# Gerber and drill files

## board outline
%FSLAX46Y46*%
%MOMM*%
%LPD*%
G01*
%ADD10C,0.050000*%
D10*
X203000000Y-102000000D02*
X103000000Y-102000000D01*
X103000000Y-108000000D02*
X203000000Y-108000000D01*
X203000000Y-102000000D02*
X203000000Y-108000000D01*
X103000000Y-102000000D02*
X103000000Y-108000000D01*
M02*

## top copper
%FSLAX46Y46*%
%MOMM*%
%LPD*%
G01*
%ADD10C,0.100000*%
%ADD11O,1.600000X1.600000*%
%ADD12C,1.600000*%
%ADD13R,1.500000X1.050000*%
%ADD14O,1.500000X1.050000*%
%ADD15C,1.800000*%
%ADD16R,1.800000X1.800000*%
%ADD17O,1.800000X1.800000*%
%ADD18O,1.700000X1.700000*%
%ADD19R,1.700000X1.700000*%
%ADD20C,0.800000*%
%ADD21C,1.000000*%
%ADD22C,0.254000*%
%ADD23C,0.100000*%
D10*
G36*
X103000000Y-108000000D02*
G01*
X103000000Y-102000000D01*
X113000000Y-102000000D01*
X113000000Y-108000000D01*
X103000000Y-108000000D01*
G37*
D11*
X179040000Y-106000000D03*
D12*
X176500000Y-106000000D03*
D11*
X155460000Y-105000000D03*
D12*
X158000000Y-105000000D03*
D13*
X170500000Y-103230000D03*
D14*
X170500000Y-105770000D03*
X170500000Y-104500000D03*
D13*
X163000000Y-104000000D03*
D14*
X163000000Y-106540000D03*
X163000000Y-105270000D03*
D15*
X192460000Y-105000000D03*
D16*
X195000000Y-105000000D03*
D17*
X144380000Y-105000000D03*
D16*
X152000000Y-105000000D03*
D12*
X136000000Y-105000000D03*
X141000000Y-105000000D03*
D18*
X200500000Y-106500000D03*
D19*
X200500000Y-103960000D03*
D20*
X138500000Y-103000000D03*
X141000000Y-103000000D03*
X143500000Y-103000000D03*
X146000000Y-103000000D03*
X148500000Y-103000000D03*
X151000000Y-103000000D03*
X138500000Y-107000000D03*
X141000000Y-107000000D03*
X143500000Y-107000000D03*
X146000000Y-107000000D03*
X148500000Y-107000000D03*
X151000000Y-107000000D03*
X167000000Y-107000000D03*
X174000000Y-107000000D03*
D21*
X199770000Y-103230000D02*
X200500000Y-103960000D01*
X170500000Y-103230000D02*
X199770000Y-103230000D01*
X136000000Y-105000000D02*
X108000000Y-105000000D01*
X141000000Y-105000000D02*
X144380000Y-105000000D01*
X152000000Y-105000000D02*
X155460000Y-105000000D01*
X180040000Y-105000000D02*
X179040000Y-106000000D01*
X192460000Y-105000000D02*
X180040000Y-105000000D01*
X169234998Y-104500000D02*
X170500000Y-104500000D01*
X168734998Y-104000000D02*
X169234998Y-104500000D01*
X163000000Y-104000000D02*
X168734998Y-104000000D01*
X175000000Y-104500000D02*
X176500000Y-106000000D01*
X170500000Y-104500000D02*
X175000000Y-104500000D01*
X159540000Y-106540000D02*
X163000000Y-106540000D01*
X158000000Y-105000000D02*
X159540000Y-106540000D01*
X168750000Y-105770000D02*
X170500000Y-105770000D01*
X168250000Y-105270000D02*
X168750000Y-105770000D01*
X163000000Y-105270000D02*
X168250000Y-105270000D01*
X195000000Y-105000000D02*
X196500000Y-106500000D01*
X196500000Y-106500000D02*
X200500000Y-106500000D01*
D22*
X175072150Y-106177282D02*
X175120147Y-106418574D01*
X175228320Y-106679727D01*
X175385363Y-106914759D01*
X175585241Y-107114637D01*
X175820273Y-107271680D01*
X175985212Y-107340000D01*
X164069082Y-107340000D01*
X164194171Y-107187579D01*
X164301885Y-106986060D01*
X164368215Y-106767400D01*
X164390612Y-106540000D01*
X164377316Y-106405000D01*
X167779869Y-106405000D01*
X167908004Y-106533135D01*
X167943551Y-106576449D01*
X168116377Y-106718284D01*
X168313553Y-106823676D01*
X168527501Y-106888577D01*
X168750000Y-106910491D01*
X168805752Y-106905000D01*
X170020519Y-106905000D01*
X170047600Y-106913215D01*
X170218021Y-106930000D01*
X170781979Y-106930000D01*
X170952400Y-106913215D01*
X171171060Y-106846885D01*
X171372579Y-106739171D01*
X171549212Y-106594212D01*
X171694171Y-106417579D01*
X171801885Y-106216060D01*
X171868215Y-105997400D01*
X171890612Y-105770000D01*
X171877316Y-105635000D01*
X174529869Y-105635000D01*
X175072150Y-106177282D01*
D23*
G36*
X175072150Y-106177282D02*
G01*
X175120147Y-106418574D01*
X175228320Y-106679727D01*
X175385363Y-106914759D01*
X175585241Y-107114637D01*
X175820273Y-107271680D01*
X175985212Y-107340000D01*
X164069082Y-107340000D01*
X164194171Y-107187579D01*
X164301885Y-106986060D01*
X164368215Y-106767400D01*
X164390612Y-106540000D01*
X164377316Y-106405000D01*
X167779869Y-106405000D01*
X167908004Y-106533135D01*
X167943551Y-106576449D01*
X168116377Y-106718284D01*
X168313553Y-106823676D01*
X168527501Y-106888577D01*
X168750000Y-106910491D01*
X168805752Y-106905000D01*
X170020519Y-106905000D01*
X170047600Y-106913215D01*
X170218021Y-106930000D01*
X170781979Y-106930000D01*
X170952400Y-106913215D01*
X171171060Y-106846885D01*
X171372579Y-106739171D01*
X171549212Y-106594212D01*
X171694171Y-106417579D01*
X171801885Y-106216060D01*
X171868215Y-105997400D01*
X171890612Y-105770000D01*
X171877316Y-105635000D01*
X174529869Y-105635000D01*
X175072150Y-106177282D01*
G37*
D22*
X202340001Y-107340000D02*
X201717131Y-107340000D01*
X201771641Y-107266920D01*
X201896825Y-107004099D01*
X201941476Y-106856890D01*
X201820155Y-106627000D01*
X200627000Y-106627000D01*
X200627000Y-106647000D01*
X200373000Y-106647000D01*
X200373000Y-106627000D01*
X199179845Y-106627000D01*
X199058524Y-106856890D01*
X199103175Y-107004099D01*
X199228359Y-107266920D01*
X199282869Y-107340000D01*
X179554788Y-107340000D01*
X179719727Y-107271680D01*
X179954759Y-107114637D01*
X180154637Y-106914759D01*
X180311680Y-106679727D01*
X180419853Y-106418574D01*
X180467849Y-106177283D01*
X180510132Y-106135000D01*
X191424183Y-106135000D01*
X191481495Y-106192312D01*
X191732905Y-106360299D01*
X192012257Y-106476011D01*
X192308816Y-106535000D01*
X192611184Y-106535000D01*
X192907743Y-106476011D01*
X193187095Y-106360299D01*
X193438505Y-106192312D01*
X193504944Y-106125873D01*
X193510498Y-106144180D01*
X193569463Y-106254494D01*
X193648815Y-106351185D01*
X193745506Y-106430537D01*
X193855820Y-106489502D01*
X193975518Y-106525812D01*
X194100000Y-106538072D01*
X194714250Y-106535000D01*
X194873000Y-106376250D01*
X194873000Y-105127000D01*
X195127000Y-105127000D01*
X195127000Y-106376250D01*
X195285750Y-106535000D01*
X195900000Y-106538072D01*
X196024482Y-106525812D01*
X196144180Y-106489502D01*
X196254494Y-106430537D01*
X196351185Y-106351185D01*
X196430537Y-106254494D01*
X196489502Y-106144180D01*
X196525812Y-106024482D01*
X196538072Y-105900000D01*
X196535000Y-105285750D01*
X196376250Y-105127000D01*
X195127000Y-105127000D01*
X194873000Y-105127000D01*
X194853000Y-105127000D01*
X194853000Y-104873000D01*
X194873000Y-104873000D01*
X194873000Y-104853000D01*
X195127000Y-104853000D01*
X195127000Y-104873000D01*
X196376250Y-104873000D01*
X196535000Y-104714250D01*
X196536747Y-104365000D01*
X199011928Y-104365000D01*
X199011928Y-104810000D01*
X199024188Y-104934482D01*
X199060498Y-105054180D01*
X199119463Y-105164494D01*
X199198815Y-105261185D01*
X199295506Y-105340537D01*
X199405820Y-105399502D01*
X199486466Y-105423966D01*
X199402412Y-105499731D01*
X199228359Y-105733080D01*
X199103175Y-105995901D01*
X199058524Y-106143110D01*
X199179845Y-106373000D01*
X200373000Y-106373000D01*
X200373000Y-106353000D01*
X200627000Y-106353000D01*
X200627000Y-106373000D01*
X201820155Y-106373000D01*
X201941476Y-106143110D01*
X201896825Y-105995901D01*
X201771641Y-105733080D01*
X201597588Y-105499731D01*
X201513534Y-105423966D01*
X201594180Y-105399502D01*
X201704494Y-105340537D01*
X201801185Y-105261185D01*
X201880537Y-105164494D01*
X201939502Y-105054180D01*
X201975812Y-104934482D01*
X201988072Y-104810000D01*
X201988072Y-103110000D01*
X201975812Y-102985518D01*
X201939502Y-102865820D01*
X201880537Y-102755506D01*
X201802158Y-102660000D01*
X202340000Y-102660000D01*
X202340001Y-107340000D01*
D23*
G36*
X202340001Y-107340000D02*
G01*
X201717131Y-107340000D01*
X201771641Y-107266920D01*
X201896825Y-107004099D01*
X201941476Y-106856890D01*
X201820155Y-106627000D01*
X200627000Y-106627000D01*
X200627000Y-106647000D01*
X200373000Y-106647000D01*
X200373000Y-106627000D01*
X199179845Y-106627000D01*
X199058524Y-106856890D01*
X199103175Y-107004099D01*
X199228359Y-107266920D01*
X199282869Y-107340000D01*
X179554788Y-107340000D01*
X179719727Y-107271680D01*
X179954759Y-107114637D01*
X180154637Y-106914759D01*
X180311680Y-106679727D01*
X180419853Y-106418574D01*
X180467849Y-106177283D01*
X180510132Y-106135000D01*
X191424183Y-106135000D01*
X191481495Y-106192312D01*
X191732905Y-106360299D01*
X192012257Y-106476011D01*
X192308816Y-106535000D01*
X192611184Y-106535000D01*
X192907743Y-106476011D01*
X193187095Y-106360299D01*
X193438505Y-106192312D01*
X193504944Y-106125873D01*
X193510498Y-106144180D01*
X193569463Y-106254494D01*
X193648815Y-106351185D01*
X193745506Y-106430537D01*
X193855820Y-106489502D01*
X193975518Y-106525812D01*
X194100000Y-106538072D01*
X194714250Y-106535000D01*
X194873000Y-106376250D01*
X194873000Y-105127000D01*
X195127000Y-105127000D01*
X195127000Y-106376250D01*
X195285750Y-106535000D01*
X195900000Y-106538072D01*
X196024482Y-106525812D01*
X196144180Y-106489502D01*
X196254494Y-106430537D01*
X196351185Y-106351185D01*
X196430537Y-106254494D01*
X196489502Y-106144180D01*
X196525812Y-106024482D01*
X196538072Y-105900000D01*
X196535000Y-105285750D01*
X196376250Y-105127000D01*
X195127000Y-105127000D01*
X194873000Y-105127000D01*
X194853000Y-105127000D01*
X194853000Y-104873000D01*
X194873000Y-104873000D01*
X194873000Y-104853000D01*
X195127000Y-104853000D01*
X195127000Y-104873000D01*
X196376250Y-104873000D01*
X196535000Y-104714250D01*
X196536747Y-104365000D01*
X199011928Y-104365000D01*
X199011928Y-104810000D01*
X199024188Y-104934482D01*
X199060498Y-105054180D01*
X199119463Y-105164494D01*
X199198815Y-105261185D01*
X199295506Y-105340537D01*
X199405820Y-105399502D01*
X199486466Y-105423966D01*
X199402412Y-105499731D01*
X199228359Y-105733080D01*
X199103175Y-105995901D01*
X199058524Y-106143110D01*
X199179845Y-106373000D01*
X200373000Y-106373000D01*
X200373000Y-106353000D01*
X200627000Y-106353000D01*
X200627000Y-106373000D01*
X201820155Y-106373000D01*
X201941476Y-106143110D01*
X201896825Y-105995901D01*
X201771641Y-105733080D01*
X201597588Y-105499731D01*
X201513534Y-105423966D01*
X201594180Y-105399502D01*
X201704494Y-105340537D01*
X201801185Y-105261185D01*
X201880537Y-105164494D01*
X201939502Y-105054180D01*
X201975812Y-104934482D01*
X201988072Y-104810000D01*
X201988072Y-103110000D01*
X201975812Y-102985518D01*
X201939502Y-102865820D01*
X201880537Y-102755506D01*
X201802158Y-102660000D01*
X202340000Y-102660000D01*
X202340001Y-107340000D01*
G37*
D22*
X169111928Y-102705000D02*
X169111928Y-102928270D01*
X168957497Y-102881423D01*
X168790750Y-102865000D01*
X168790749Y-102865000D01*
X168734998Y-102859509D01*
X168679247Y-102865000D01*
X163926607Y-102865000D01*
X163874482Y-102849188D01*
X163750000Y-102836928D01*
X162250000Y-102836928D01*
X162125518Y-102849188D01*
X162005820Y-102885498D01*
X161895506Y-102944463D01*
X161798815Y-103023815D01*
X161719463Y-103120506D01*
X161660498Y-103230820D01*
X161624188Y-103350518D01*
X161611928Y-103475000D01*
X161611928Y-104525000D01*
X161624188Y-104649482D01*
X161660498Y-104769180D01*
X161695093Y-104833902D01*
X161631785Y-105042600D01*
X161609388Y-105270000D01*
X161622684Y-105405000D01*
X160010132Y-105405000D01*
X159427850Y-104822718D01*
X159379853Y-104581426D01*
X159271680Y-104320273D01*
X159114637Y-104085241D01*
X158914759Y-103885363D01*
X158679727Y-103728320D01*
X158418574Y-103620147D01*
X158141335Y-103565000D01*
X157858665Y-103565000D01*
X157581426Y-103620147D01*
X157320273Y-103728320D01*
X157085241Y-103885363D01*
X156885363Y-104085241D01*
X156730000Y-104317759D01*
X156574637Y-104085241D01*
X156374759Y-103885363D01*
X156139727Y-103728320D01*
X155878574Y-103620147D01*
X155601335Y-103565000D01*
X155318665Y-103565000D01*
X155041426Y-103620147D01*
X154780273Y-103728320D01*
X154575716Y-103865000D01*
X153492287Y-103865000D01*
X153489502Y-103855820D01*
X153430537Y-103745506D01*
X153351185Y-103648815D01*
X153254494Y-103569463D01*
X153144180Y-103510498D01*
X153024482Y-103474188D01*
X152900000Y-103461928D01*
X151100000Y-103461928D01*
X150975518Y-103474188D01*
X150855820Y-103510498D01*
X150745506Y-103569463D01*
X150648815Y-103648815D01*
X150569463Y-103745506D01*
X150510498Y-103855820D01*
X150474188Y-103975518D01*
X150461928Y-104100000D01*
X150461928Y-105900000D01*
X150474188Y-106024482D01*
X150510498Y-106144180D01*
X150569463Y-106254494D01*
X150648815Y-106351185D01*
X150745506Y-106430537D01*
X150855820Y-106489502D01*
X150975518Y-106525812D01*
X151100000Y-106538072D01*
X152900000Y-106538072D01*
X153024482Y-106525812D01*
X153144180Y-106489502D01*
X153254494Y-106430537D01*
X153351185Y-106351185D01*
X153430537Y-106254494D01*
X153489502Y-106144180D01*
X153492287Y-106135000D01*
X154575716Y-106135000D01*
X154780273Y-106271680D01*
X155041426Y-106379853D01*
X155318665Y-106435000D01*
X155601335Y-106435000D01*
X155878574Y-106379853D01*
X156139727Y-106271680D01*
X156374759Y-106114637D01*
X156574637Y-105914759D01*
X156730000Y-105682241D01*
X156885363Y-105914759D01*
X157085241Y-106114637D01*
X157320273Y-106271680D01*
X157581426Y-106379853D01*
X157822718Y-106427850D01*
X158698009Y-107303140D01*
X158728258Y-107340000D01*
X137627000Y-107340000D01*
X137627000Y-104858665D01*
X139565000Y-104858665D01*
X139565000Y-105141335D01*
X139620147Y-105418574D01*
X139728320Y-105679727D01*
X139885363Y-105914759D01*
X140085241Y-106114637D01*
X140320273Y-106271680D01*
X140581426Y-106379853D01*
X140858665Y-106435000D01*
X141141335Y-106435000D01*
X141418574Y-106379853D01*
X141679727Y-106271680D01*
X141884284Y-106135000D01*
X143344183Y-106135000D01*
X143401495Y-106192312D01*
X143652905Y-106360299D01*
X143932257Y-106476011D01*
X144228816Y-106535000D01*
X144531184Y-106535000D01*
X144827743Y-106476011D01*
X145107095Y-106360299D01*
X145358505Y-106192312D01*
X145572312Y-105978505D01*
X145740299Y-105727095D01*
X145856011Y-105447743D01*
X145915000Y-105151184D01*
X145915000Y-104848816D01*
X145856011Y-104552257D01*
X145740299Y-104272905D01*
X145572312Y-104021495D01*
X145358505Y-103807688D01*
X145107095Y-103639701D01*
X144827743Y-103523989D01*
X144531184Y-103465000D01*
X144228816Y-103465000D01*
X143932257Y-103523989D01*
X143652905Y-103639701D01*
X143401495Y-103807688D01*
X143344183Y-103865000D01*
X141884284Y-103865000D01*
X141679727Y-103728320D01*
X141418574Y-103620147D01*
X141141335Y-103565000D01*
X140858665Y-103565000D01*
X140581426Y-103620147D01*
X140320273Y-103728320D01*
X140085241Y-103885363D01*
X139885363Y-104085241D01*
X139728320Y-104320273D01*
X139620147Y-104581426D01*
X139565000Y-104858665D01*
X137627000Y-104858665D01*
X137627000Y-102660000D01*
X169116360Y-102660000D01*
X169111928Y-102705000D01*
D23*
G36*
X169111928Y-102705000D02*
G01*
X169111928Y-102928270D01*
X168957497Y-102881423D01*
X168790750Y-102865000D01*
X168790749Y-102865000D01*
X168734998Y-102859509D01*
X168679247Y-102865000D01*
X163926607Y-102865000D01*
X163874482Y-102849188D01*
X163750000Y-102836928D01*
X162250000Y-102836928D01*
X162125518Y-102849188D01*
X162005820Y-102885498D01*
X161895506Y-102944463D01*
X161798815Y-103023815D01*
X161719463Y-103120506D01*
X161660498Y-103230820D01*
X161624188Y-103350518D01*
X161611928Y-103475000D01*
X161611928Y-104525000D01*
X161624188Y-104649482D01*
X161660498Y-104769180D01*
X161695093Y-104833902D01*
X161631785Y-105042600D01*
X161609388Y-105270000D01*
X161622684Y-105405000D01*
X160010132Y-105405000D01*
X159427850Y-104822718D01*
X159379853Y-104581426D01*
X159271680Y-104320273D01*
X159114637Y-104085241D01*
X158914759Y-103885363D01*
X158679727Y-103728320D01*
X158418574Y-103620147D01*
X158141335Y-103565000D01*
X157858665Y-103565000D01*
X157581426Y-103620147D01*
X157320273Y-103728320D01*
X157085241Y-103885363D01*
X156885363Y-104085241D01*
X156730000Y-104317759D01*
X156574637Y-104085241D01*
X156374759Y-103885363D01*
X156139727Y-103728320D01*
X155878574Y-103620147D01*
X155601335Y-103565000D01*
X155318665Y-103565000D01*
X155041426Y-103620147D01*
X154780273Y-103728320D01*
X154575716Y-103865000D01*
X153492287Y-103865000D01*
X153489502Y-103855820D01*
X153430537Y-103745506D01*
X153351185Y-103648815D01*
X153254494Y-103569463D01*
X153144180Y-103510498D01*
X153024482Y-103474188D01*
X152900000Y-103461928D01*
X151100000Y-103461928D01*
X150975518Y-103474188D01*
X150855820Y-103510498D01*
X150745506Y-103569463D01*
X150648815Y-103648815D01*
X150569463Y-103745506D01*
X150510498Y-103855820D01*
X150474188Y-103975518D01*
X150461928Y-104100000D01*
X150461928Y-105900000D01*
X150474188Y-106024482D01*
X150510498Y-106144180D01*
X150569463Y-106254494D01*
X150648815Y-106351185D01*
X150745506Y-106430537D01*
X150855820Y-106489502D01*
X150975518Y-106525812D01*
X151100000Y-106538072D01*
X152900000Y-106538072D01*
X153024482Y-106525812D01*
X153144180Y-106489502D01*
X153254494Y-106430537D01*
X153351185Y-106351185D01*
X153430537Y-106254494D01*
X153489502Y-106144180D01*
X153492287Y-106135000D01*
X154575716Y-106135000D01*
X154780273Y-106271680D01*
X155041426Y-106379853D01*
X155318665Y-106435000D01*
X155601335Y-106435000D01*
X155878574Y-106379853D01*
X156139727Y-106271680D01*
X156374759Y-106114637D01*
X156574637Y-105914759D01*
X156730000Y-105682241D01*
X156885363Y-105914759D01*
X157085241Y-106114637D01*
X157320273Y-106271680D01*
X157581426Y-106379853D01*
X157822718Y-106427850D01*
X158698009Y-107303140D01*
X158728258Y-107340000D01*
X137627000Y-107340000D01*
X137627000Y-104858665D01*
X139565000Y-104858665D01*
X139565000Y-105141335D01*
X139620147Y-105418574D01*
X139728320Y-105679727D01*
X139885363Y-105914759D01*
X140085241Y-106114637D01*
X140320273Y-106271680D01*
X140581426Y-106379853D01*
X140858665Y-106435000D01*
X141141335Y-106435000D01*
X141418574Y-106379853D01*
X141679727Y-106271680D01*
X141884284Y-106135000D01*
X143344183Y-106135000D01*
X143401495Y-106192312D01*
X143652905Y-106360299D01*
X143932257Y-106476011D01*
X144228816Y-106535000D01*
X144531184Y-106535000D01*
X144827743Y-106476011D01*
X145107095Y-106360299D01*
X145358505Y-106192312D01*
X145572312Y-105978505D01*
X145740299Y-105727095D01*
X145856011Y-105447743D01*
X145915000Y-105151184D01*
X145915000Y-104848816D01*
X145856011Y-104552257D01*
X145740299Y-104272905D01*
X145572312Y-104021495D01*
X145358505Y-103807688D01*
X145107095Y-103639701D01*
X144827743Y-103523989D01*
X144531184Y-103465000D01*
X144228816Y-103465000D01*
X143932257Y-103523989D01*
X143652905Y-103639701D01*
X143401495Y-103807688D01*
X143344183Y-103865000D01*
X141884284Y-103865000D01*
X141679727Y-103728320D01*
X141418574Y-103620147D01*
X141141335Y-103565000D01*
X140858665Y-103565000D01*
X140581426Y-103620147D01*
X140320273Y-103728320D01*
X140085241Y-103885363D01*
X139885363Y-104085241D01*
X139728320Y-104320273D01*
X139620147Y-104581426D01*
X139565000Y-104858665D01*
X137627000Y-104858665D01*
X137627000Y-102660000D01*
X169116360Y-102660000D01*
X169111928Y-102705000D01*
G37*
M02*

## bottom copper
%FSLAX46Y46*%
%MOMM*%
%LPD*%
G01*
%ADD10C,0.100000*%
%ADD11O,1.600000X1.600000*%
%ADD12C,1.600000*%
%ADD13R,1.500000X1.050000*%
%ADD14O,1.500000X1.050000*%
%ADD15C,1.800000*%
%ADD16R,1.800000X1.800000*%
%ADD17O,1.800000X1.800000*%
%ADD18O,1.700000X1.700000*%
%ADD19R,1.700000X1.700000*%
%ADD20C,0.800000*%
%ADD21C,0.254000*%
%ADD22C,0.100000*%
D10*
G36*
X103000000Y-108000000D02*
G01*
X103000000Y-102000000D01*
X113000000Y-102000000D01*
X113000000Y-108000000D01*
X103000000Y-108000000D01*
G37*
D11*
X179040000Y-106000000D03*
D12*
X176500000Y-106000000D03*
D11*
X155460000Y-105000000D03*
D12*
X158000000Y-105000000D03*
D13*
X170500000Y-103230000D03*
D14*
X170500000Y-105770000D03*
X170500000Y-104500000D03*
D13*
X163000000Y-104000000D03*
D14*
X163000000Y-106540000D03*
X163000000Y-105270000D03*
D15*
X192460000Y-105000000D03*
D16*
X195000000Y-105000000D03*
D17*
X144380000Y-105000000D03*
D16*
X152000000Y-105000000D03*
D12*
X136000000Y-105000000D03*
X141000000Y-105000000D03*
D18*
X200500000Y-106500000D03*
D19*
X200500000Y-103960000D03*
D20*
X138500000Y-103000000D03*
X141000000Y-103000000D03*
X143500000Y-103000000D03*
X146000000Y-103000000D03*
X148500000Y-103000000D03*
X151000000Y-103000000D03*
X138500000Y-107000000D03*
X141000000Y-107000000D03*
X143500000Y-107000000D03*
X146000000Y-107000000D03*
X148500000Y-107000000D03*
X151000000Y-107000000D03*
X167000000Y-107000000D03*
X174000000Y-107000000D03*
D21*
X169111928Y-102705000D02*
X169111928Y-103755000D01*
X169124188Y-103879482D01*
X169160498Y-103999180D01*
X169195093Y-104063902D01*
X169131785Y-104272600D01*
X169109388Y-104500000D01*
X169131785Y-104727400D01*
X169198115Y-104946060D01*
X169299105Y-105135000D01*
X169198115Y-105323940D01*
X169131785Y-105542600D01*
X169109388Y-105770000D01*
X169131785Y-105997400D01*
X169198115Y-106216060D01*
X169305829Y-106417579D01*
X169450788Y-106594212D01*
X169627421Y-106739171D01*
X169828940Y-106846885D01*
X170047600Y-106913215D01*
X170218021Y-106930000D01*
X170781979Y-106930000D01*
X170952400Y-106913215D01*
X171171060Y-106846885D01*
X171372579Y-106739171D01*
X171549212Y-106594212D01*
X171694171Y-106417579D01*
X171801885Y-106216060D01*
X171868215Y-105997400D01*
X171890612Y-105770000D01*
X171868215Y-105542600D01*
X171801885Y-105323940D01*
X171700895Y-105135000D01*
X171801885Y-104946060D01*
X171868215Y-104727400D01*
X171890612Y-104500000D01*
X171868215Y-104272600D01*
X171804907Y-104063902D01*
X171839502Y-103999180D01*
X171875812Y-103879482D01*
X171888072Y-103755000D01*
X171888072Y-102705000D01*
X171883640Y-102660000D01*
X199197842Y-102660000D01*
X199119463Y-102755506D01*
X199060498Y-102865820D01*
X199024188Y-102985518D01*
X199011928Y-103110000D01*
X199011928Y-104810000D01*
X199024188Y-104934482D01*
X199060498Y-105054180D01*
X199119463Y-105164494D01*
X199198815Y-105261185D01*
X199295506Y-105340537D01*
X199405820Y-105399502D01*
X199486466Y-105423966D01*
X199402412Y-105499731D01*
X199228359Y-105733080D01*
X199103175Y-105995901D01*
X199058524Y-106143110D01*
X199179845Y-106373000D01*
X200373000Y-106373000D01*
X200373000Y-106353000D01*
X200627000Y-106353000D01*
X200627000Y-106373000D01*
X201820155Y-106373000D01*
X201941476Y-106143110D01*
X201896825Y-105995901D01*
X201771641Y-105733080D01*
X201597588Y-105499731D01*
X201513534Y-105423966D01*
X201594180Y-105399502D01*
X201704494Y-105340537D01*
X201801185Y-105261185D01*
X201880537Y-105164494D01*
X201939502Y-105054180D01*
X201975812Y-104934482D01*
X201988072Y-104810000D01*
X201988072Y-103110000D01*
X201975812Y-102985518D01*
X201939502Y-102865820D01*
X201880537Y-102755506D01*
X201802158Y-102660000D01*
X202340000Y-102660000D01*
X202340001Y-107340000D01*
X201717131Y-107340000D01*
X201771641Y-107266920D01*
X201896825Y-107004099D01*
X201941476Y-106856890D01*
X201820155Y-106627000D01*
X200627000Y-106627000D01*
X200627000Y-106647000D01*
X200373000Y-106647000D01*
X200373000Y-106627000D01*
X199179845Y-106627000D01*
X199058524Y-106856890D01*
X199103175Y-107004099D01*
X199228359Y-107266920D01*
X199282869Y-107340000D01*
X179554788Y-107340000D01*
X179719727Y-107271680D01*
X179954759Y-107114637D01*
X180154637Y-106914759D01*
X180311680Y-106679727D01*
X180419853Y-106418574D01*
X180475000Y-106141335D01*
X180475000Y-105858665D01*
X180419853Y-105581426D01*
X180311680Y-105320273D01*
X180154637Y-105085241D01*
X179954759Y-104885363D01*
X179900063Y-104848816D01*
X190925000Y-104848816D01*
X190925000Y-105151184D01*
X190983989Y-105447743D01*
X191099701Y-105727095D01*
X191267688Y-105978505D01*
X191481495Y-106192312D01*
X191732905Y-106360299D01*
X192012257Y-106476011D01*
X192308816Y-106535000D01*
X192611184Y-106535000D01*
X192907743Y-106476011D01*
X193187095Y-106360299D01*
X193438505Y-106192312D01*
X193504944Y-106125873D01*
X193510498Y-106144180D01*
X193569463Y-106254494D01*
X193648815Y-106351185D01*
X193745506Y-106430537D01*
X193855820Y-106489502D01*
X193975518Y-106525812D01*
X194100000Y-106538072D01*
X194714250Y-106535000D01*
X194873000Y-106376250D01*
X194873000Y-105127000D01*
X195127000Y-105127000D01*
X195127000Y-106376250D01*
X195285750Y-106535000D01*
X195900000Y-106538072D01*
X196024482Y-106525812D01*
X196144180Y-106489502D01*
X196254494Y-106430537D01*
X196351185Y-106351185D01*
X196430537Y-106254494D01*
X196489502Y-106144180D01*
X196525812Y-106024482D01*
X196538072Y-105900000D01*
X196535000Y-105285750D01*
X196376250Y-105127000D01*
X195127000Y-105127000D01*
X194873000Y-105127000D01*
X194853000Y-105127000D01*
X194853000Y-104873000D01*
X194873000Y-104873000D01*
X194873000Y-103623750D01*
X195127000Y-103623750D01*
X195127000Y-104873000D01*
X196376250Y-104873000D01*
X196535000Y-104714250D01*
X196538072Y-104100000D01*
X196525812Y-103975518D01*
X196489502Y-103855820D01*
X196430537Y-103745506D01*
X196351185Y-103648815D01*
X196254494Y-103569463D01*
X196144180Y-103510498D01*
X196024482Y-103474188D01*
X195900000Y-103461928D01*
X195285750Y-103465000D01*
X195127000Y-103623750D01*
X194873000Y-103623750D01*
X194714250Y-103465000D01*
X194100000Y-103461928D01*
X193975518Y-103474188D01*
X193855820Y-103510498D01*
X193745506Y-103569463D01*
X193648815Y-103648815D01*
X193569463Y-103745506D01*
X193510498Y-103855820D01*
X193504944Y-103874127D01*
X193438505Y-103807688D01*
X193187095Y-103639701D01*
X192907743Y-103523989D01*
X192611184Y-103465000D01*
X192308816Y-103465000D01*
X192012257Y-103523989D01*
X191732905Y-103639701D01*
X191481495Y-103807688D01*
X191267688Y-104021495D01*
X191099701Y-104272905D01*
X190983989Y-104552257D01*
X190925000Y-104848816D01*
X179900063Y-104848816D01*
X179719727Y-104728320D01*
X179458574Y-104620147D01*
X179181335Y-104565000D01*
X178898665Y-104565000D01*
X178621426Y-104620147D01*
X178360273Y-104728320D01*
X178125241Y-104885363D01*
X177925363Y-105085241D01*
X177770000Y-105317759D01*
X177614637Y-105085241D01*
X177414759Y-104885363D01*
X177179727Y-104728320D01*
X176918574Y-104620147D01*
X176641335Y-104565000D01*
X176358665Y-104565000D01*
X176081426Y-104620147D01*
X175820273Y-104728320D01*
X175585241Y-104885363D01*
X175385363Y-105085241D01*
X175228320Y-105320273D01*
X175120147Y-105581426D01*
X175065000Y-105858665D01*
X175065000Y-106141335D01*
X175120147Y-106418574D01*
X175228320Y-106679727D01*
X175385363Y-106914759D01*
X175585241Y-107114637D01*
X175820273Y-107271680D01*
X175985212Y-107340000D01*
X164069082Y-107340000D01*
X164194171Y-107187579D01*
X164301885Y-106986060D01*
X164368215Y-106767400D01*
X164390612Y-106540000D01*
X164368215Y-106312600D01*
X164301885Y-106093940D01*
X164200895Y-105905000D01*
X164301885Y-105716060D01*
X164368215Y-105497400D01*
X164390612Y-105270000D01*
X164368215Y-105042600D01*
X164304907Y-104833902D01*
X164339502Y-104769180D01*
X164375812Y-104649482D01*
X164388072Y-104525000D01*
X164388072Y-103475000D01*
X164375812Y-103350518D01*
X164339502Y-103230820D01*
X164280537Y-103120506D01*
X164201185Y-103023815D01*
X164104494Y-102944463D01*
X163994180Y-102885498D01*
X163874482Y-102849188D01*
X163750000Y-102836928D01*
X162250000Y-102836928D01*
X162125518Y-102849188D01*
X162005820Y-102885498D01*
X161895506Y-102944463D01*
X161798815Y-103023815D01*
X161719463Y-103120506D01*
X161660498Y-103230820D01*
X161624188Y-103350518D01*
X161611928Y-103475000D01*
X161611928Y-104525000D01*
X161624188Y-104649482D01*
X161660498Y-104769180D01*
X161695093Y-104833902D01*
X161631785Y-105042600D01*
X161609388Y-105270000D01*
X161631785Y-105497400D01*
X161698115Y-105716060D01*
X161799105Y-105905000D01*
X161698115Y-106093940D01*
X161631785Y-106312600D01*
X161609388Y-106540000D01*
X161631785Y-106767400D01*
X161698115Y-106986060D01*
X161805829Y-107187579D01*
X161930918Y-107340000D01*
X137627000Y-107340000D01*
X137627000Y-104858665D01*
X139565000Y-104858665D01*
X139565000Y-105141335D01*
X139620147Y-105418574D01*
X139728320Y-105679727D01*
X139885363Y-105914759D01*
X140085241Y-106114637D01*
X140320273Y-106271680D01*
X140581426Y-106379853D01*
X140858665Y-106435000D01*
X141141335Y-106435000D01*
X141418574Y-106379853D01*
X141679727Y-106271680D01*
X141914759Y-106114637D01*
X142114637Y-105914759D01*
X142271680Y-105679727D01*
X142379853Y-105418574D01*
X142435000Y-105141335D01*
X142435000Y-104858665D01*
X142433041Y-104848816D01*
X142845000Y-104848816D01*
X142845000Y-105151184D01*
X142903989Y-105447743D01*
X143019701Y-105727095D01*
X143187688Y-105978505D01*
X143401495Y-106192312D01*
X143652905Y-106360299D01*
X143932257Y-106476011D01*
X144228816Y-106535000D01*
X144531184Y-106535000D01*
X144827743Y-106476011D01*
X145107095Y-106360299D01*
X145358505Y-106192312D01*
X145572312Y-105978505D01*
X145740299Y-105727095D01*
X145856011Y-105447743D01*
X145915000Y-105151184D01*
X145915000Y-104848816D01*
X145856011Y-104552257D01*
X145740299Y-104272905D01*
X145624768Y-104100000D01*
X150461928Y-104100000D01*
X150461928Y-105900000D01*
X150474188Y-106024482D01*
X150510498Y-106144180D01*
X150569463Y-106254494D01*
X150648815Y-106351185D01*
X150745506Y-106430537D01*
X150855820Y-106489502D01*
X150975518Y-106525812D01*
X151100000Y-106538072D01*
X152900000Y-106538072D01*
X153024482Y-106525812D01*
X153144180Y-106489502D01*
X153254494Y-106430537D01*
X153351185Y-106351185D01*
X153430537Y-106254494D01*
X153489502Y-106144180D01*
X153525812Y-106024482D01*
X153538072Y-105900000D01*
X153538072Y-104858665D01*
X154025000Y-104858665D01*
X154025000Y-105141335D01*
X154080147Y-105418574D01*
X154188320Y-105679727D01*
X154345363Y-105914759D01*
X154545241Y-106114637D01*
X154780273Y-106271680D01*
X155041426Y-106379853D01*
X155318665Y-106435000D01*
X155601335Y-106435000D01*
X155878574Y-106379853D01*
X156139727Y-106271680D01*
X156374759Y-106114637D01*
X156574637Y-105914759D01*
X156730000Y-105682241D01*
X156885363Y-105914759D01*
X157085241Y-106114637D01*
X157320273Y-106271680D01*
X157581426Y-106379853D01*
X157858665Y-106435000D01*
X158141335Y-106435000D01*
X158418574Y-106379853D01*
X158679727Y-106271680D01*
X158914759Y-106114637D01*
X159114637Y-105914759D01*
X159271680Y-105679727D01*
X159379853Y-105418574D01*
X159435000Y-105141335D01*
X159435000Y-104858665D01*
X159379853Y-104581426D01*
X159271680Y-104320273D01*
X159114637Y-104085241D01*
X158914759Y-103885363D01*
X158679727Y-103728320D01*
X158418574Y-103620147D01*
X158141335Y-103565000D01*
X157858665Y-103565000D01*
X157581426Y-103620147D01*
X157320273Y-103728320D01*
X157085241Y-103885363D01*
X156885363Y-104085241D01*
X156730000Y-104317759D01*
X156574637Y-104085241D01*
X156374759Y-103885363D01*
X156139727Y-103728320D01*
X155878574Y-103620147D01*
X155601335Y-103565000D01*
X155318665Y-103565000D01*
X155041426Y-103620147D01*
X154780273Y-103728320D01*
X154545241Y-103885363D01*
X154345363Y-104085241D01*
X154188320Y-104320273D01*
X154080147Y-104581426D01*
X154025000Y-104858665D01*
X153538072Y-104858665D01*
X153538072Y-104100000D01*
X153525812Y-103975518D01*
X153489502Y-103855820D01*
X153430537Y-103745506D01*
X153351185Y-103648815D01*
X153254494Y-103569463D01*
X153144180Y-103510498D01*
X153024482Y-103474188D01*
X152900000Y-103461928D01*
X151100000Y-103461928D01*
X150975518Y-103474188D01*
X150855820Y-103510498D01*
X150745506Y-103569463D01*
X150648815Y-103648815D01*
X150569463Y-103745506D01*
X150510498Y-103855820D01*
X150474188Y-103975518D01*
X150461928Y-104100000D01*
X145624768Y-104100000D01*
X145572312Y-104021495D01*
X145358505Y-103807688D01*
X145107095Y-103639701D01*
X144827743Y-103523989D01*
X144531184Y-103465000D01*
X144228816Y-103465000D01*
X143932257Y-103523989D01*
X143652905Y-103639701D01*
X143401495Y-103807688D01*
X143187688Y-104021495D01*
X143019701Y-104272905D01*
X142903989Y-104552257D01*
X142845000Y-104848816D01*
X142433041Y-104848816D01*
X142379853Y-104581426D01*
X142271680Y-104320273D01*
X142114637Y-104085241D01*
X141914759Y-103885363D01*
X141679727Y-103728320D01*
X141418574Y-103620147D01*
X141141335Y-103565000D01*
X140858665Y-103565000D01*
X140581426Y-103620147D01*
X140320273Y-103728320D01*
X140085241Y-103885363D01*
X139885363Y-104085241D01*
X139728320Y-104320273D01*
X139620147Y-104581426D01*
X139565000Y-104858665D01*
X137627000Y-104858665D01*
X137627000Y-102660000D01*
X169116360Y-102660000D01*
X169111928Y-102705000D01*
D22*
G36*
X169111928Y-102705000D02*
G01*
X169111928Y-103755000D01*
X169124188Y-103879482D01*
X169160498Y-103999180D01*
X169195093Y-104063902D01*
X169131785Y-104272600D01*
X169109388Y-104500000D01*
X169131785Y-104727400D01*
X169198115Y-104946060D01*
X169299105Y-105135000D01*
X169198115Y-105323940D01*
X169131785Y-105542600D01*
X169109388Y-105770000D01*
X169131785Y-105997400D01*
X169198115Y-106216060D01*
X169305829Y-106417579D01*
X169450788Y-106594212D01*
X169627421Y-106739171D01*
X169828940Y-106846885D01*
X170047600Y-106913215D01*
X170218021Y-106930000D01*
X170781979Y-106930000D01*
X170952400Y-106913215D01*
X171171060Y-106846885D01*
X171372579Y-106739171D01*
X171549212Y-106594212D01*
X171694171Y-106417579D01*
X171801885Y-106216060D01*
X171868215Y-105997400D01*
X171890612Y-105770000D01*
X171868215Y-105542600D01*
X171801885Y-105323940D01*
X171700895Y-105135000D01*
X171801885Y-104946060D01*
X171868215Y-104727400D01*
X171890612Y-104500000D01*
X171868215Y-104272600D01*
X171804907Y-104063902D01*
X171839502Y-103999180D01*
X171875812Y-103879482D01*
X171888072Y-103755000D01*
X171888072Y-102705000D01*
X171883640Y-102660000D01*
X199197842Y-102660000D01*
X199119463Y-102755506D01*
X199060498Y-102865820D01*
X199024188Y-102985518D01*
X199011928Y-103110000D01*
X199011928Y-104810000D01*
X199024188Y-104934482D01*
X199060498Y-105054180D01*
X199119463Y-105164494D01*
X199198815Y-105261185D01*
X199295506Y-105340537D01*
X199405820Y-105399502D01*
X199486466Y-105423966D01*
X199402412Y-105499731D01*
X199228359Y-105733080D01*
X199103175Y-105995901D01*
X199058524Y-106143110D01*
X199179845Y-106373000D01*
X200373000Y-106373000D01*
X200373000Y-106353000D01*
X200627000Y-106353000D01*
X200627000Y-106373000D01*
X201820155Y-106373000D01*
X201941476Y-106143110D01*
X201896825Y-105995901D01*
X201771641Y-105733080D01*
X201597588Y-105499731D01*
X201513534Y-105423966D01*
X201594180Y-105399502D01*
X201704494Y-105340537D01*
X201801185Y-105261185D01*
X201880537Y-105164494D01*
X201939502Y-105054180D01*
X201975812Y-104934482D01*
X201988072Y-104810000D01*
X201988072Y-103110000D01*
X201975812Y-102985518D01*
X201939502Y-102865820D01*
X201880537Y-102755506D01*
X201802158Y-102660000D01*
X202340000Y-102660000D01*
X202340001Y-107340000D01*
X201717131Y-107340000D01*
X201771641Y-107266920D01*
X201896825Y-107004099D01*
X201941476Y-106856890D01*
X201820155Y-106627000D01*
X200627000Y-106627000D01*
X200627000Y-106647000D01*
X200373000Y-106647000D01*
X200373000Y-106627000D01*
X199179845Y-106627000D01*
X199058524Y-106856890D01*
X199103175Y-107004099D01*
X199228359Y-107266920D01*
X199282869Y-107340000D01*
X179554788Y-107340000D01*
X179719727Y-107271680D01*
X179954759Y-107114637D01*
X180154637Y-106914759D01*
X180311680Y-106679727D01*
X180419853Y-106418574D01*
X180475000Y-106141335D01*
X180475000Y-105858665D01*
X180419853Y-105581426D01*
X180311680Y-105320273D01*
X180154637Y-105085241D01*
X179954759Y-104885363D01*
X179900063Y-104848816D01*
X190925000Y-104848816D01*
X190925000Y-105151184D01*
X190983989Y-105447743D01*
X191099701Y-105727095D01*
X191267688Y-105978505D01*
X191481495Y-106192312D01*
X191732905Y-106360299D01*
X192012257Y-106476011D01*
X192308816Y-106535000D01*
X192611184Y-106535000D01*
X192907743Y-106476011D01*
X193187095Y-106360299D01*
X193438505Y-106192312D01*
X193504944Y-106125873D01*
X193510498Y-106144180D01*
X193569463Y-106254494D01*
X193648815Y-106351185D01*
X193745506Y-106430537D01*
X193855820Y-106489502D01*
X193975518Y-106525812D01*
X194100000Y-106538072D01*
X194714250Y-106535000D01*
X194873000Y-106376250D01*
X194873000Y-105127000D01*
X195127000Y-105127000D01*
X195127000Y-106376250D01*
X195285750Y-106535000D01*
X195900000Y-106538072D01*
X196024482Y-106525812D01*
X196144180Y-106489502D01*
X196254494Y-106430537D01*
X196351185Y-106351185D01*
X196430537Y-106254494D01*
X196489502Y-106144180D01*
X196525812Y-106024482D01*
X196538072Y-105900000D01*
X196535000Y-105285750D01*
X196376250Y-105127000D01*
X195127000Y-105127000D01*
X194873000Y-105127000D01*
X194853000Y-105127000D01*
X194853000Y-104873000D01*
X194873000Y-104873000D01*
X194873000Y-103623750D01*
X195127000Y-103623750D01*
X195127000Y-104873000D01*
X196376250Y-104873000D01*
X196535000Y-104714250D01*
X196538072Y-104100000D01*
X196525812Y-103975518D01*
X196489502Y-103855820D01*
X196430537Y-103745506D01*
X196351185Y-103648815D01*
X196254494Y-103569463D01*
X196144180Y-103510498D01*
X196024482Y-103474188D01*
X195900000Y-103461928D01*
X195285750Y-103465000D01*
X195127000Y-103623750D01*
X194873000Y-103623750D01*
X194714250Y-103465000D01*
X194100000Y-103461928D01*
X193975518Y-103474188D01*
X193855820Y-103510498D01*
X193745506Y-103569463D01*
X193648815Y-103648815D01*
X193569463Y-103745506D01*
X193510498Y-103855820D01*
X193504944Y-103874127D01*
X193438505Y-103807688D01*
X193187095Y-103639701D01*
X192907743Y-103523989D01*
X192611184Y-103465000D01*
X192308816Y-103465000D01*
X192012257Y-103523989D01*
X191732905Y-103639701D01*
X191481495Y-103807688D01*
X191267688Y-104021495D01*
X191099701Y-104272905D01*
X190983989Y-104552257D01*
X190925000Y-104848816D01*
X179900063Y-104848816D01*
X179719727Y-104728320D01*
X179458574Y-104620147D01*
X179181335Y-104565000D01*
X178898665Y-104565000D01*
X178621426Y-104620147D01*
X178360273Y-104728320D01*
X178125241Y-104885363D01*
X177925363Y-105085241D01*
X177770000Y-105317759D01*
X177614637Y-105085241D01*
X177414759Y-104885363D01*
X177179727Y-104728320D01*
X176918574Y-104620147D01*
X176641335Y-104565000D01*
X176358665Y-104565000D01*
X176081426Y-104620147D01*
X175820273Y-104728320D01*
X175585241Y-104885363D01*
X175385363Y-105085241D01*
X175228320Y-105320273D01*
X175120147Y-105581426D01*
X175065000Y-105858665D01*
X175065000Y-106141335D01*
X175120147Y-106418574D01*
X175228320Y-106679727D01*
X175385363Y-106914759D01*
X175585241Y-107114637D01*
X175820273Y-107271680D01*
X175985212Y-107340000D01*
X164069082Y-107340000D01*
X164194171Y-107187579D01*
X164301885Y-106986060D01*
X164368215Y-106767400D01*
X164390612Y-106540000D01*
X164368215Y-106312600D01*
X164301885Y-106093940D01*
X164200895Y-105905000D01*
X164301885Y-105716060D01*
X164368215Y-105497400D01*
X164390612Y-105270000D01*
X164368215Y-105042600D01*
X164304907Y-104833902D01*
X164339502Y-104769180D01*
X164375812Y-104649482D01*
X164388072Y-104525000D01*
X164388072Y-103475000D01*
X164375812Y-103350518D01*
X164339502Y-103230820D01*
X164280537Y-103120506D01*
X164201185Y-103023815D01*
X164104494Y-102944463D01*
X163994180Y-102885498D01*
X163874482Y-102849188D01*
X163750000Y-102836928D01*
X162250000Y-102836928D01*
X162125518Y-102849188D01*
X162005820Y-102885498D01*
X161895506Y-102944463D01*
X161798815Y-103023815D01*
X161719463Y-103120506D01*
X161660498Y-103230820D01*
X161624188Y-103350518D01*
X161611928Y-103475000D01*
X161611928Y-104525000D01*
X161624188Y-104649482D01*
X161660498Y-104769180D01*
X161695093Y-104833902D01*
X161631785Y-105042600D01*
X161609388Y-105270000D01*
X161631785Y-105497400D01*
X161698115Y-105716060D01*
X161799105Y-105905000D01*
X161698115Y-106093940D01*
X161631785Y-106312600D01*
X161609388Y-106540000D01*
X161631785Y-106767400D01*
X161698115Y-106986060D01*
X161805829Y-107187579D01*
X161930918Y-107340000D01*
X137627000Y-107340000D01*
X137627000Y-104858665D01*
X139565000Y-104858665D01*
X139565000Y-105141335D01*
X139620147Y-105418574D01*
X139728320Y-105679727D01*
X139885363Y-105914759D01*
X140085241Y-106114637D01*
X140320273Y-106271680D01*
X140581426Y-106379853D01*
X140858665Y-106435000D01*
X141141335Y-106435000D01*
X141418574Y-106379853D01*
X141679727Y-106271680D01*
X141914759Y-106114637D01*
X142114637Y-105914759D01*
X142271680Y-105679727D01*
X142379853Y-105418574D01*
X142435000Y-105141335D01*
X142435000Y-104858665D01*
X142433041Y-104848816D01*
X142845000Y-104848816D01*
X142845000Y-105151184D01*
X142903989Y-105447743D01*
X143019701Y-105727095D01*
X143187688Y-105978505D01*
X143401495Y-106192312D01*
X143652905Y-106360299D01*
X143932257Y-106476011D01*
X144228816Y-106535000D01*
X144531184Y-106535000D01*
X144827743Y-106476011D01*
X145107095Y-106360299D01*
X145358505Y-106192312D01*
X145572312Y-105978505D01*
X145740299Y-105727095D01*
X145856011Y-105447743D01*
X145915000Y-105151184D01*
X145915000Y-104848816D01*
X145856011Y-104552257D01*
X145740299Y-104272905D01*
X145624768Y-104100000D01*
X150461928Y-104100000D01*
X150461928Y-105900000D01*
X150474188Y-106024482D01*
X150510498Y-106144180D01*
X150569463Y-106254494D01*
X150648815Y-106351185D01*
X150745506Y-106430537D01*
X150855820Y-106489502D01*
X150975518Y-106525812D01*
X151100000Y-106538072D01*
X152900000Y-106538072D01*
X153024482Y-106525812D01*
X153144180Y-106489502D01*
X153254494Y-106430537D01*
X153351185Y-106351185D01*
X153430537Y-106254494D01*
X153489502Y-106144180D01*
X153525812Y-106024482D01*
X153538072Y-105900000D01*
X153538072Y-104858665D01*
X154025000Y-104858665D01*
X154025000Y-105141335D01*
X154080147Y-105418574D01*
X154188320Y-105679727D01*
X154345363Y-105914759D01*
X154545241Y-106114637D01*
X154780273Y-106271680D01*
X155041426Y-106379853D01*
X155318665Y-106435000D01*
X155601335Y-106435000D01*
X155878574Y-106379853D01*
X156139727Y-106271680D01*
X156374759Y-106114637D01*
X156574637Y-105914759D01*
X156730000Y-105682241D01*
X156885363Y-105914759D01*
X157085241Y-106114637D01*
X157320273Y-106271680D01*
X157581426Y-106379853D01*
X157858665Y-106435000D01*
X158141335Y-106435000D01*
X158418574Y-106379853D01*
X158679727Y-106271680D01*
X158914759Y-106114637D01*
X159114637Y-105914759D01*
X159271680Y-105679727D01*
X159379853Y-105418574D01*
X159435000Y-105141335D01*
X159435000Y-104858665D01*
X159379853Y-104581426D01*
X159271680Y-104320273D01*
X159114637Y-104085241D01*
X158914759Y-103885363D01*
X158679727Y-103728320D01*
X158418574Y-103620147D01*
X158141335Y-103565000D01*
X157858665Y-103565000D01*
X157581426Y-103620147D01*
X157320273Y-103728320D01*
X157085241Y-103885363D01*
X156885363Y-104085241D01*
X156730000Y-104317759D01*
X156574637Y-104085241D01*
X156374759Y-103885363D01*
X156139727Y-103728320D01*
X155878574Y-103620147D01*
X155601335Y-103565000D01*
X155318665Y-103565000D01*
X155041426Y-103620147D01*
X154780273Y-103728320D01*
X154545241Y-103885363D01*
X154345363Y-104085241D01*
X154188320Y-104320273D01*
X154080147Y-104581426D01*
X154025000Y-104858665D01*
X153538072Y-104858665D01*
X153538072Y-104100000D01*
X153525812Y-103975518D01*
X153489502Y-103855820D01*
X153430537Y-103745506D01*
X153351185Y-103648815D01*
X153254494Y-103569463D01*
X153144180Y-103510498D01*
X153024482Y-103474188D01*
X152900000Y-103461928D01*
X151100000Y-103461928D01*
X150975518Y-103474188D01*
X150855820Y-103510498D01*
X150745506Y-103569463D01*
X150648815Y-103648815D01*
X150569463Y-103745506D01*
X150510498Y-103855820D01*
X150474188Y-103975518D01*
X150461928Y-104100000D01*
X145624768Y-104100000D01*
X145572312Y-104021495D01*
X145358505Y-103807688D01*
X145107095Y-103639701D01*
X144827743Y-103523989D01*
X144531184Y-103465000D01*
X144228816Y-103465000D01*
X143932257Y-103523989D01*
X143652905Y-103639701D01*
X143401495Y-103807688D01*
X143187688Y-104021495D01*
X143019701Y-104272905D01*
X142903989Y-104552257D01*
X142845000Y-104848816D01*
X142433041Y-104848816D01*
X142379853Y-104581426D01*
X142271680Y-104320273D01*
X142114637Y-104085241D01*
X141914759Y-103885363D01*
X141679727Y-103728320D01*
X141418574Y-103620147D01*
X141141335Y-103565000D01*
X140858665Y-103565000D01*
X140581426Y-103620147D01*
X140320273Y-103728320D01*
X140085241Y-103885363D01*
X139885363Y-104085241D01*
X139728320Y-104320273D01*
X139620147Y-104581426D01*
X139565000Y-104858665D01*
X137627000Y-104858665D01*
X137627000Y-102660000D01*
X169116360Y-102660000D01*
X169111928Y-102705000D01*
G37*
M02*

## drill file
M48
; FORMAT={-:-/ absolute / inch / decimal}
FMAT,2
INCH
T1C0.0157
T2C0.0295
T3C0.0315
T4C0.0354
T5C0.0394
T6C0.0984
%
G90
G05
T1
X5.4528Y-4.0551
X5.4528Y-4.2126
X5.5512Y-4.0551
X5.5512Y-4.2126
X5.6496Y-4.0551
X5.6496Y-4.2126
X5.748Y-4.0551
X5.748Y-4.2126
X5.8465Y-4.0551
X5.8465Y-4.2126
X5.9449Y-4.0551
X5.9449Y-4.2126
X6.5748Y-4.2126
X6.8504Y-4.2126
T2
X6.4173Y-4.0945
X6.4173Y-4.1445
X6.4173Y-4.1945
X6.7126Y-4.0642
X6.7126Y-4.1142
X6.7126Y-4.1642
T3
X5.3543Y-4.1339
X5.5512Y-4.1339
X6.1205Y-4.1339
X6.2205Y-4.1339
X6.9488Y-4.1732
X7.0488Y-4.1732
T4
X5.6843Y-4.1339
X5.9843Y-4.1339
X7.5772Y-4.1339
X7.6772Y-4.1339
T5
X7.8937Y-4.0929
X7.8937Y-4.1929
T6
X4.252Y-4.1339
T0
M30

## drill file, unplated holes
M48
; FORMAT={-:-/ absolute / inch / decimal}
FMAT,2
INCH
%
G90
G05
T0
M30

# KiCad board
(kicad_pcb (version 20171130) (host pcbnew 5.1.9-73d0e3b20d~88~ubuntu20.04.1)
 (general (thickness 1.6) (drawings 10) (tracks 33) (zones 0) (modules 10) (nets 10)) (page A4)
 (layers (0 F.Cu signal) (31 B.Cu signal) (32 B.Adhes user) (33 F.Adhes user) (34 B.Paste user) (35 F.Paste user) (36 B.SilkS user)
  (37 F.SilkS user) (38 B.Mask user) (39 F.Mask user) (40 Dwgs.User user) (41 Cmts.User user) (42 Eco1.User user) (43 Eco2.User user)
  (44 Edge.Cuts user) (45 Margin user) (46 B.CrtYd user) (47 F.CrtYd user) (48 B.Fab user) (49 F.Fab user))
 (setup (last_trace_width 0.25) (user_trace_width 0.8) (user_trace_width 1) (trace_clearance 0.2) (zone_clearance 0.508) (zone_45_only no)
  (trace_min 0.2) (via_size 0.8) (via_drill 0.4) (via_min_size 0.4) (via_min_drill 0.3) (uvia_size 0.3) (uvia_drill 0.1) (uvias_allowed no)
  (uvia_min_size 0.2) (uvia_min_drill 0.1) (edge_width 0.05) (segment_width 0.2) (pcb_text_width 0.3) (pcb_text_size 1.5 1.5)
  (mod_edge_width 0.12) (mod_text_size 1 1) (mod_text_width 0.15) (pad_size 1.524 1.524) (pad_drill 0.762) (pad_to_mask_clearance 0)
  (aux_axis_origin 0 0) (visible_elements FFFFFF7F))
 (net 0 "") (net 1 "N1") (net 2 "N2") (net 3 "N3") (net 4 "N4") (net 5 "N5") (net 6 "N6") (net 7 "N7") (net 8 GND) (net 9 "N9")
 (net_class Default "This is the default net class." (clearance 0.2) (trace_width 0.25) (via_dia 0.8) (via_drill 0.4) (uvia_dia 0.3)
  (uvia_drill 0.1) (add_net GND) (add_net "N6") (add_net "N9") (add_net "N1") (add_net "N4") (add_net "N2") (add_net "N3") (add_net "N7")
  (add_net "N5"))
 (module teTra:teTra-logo (layer B.Cu) (at 185.2 104.8)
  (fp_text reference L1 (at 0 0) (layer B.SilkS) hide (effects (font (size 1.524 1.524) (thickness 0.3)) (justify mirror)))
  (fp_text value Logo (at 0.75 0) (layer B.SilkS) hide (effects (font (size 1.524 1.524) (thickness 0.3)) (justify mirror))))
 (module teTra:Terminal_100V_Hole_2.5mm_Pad (layer F.Cu) (at 108 105)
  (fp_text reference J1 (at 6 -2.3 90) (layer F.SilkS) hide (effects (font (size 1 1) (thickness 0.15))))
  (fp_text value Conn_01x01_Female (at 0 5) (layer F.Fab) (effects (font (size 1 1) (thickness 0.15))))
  (pad 1 thru_hole trapezoid (at 0 0) (size 10 6) (drill 2.5) (layers *.Cu *.Mask) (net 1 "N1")))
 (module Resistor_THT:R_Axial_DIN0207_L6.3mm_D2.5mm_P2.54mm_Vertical (layer F.Cu) (at 176.5 106)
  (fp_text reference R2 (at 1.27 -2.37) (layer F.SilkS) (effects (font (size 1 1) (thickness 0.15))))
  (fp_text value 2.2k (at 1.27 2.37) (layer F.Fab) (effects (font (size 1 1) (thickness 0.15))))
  (pad 2 thru_hole oval (at 2.54 0) (size 1.6 1.6) (drill 0.8) (layers *.Cu *.Mask) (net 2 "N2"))
  (pad 1 thru_hole circle (at 0 0) (size 1.6 1.6) (drill 0.8) (layers *.Cu *.Mask) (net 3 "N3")))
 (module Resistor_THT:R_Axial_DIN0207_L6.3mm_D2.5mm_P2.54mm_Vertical (layer F.Cu) (at 158 105 180)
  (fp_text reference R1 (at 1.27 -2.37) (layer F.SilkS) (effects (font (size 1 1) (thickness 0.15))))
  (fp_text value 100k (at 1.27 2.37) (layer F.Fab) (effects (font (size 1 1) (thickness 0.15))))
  (pad 2 thru_hole oval (at 2.54 0 180) (size 1.6 1.6) (drill 0.8) (layers *.Cu *.Mask) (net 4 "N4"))
  (pad 1 thru_hole circle (at 0 0 180) (size 1.6 1.6) (drill 0.8) (layers *.Cu *.Mask) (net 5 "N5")))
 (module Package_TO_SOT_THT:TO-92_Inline (layer F.Cu) (at 170.5 103.23 270)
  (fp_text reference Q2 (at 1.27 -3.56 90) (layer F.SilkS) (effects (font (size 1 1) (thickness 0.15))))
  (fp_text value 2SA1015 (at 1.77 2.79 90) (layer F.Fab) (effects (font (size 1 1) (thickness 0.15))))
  (pad 1 thru_hole rect (at 0 0 270) (size 1.05 1.5) (drill 0.75) (layers *.Cu *.Mask) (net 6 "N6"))
  (pad 3 thru_hole oval (at 2.54 0 270) (size 1.05 1.5) (drill 0.75) (layers *.Cu *.Mask) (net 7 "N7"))
  (pad 2 thru_hole oval (at 1.27 0 270) (size 1.05 1.5) (drill 0.75) (layers *.Cu *.Mask) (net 3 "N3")))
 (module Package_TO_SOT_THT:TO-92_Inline (layer F.Cu) (at 163 104 270)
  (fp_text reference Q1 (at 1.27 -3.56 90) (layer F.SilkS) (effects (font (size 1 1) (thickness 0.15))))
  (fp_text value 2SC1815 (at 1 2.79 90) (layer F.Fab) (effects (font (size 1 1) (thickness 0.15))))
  (pad 1 thru_hole rect (at 0 0 270) (size 1.05 1.5) (drill 0.75) (layers *.Cu *.Mask) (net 3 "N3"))
  (pad 3 thru_hole oval (at 2.54 0 270) (size 1.05 1.5) (drill 0.75) (layers *.Cu *.Mask) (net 5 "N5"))
  (pad 2 thru_hole oval (at 1.27 0 270) (size 1.05 1.5) (drill 0.75) (layers *.Cu *.Mask) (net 7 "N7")))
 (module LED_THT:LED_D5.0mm (layer F.Cu) (at 195 105 180)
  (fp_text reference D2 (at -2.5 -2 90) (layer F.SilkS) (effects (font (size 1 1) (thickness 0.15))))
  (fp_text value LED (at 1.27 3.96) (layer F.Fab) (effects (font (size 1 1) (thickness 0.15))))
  (pad 2 thru_hole circle (at 2.54 0 180) (size 1.8 1.8) (drill 0.9) (layers *.Cu *.Mask) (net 2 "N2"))
  (pad 1 thru_hole rect (at 0 0 180) (size 1.8 1.8) (drill 0.9) (layers *.Cu *.Mask) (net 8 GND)))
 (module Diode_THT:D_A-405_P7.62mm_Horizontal (layer F.Cu) (at 152 105 180)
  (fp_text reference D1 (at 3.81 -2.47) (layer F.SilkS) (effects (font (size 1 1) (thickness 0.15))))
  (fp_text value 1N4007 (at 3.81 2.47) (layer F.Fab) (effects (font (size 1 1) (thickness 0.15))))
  (pad 2 thru_hole oval (at 7.62 0 180) (size 1.8 1.8) (drill 0.9) (layers *.Cu *.Mask) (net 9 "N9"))
  (pad 1 thru_hole rect (at 0 0 180) (size 1.8 1.8) (drill 0.9) (layers *.Cu *.Mask) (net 4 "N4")))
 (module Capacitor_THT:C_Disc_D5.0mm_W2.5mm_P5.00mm (layer F.Cu) (at 141 105 180)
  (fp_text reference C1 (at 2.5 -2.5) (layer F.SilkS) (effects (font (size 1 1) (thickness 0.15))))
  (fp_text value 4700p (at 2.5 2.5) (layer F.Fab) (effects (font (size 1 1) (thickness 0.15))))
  (pad 2 thru_hole circle (at 5 0 180) (size 1.6 1.6) (drill 0.8) (layers *.Cu *.Mask) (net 1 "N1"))
  (pad 1 thru_hole circle (at 0 0 180) (size 1.6 1.6) (drill 0.8) (layers *.Cu *.Mask) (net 9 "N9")))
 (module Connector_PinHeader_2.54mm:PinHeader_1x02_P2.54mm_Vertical (layer F.Cu) (at 200.5 103.96)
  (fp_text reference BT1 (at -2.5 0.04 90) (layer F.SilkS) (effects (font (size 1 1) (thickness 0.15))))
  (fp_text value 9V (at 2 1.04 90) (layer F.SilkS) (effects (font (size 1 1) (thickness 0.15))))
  (pad 2 thru_hole oval (at 0 2.54) (size 1.7 1.7) (drill 1) (layers *.Cu *.Mask) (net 8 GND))
  (pad 1 thru_hole rect (at 0 0) (size 1.7 1.7) (drill 1) (layers *.Cu *.Mask) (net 6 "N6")))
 (gr_line (start 203 102) (end 103 102) (layer Edge.Cuts) (width 0.05))
 (gr_line (start 103 108) (end 203 108) (layer Edge.Cuts) (width 0.05))
 (gr_line (start 203 102) (end 203 108) (layer Edge.Cuts) (width 0.05))
 (gr_line (start 103 102) (end 103 108) (layer Edge.Cuts) (width 0.05))
 (segment (start 199.77 103.23) (end 200.5 103.96) (width 1) (layer F.Cu) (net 6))
 (segment (start 170.5 103.23) (end 199.77 103.23) (width 1) (layer F.Cu) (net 6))
 (segment (start 136 105) (end 108 105) (width 1) (layer F.Cu) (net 1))
 (segment (start 141 105) (end 144.38 105) (width 1) (layer F.Cu) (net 9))
 (segment (start 152 105) (end 155.46 105) (width 1) (layer F.Cu) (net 4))
 (segment (start 180.04 105) (end 179.04 106) (width 1) (layer F.Cu) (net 2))
 (segment (start 192.46 105) (end 180.04 105) (width 1) (layer F.Cu) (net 2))
 (segment (start 169.234998 104.5) (end 170.5 104.5) (width 1) (layer F.Cu) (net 3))
 (segment (start 168.734998 104) (end 169.234998 104.5) (width 1) (layer F.Cu) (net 3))
 (segment (start 163 104) (end 168.734998 104) (width 1) (layer F.Cu) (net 3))
 (segment (start 175 104.5) (end 176.5 106) (width 1) (layer F.Cu) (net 3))
 (segment (start 170.5 104.5) (end 175 104.5) (width 1) (layer F.Cu) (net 3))
 (segment (start 159.54 106.54) (end 163 106.54) (width 1) (layer F.Cu) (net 5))
 (segment (start 158 105) (end 159.54 106.54) (width 1) (layer F.Cu) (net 5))
 (segment (start 168.75 105.77) (end 170.5 105.77) (width 1) (layer F.Cu) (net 7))
 (segment (start 168.25 105.27) (end 168.75 105.77) (width 1) (layer F.Cu) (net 7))
 (segment (start 163 105.27) (end 168.25 105.27) (width 1) (layer F.Cu) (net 7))
 (segment (start 195 105) (end 196.5 106.5) (width 1) (layer F.Cu) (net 8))
 (segment (start 196.5 106.5) (end 200.5 106.5) (width 1) (layer F.Cu) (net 8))
 (via (at 138.5 103) (size 0.8) (drill 0.4) (layers F.Cu B.Cu) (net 8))
 (via (at 141 103) (size 0.8) (drill 0.4) (layers F.Cu B.Cu) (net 8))
 (via (at 143.5 103) (size 0.8) (drill 0.4) (layers F.Cu B.Cu) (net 8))
 (via (at 146 103) (size 0.8) (drill 0.4) (layers F.Cu B.Cu) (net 8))
 (via (at 148.5 103) (size 0.8) (drill 0.4) (layers F.Cu B.Cu) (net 8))
 (via (at 151 103) (size 0.8) (drill 0.4) (layers F.Cu B.Cu) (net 8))
 (via (at 138.5 107) (size 0.8) (drill 0.4) (layers F.Cu B.Cu) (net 8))
 (via (at 141 107) (size 0.8) (drill 0.4) (layers F.Cu B.Cu) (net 8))
 (via (at 143.5 107) (size 0.8) (drill 0.4) (layers F.Cu B.Cu) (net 8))
 (via (at 146 107) (size 0.8) (drill 0.4) (layers F.Cu B.Cu) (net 8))
 (via (at 148.5 107) (size 0.8) (drill 0.4) (layers F.Cu B.Cu) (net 8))
 (via (at 151 107) (size 0.8) (drill 0.4) (layers F.Cu B.Cu) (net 8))
 (via (at 167 107) (size 0.8) (drill 0.4) (layers F.Cu B.Cu) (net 8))
 (via (at 174 107) (size 0.8) (drill 0.4) (layers F.Cu B.Cu) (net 8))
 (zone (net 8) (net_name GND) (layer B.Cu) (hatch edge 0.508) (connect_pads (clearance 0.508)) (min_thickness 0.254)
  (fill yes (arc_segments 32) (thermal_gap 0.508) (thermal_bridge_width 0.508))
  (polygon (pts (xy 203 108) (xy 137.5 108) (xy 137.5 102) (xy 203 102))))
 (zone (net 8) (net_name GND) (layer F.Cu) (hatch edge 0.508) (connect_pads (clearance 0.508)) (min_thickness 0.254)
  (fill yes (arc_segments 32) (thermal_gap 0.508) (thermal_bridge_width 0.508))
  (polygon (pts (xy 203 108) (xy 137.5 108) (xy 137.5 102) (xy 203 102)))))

